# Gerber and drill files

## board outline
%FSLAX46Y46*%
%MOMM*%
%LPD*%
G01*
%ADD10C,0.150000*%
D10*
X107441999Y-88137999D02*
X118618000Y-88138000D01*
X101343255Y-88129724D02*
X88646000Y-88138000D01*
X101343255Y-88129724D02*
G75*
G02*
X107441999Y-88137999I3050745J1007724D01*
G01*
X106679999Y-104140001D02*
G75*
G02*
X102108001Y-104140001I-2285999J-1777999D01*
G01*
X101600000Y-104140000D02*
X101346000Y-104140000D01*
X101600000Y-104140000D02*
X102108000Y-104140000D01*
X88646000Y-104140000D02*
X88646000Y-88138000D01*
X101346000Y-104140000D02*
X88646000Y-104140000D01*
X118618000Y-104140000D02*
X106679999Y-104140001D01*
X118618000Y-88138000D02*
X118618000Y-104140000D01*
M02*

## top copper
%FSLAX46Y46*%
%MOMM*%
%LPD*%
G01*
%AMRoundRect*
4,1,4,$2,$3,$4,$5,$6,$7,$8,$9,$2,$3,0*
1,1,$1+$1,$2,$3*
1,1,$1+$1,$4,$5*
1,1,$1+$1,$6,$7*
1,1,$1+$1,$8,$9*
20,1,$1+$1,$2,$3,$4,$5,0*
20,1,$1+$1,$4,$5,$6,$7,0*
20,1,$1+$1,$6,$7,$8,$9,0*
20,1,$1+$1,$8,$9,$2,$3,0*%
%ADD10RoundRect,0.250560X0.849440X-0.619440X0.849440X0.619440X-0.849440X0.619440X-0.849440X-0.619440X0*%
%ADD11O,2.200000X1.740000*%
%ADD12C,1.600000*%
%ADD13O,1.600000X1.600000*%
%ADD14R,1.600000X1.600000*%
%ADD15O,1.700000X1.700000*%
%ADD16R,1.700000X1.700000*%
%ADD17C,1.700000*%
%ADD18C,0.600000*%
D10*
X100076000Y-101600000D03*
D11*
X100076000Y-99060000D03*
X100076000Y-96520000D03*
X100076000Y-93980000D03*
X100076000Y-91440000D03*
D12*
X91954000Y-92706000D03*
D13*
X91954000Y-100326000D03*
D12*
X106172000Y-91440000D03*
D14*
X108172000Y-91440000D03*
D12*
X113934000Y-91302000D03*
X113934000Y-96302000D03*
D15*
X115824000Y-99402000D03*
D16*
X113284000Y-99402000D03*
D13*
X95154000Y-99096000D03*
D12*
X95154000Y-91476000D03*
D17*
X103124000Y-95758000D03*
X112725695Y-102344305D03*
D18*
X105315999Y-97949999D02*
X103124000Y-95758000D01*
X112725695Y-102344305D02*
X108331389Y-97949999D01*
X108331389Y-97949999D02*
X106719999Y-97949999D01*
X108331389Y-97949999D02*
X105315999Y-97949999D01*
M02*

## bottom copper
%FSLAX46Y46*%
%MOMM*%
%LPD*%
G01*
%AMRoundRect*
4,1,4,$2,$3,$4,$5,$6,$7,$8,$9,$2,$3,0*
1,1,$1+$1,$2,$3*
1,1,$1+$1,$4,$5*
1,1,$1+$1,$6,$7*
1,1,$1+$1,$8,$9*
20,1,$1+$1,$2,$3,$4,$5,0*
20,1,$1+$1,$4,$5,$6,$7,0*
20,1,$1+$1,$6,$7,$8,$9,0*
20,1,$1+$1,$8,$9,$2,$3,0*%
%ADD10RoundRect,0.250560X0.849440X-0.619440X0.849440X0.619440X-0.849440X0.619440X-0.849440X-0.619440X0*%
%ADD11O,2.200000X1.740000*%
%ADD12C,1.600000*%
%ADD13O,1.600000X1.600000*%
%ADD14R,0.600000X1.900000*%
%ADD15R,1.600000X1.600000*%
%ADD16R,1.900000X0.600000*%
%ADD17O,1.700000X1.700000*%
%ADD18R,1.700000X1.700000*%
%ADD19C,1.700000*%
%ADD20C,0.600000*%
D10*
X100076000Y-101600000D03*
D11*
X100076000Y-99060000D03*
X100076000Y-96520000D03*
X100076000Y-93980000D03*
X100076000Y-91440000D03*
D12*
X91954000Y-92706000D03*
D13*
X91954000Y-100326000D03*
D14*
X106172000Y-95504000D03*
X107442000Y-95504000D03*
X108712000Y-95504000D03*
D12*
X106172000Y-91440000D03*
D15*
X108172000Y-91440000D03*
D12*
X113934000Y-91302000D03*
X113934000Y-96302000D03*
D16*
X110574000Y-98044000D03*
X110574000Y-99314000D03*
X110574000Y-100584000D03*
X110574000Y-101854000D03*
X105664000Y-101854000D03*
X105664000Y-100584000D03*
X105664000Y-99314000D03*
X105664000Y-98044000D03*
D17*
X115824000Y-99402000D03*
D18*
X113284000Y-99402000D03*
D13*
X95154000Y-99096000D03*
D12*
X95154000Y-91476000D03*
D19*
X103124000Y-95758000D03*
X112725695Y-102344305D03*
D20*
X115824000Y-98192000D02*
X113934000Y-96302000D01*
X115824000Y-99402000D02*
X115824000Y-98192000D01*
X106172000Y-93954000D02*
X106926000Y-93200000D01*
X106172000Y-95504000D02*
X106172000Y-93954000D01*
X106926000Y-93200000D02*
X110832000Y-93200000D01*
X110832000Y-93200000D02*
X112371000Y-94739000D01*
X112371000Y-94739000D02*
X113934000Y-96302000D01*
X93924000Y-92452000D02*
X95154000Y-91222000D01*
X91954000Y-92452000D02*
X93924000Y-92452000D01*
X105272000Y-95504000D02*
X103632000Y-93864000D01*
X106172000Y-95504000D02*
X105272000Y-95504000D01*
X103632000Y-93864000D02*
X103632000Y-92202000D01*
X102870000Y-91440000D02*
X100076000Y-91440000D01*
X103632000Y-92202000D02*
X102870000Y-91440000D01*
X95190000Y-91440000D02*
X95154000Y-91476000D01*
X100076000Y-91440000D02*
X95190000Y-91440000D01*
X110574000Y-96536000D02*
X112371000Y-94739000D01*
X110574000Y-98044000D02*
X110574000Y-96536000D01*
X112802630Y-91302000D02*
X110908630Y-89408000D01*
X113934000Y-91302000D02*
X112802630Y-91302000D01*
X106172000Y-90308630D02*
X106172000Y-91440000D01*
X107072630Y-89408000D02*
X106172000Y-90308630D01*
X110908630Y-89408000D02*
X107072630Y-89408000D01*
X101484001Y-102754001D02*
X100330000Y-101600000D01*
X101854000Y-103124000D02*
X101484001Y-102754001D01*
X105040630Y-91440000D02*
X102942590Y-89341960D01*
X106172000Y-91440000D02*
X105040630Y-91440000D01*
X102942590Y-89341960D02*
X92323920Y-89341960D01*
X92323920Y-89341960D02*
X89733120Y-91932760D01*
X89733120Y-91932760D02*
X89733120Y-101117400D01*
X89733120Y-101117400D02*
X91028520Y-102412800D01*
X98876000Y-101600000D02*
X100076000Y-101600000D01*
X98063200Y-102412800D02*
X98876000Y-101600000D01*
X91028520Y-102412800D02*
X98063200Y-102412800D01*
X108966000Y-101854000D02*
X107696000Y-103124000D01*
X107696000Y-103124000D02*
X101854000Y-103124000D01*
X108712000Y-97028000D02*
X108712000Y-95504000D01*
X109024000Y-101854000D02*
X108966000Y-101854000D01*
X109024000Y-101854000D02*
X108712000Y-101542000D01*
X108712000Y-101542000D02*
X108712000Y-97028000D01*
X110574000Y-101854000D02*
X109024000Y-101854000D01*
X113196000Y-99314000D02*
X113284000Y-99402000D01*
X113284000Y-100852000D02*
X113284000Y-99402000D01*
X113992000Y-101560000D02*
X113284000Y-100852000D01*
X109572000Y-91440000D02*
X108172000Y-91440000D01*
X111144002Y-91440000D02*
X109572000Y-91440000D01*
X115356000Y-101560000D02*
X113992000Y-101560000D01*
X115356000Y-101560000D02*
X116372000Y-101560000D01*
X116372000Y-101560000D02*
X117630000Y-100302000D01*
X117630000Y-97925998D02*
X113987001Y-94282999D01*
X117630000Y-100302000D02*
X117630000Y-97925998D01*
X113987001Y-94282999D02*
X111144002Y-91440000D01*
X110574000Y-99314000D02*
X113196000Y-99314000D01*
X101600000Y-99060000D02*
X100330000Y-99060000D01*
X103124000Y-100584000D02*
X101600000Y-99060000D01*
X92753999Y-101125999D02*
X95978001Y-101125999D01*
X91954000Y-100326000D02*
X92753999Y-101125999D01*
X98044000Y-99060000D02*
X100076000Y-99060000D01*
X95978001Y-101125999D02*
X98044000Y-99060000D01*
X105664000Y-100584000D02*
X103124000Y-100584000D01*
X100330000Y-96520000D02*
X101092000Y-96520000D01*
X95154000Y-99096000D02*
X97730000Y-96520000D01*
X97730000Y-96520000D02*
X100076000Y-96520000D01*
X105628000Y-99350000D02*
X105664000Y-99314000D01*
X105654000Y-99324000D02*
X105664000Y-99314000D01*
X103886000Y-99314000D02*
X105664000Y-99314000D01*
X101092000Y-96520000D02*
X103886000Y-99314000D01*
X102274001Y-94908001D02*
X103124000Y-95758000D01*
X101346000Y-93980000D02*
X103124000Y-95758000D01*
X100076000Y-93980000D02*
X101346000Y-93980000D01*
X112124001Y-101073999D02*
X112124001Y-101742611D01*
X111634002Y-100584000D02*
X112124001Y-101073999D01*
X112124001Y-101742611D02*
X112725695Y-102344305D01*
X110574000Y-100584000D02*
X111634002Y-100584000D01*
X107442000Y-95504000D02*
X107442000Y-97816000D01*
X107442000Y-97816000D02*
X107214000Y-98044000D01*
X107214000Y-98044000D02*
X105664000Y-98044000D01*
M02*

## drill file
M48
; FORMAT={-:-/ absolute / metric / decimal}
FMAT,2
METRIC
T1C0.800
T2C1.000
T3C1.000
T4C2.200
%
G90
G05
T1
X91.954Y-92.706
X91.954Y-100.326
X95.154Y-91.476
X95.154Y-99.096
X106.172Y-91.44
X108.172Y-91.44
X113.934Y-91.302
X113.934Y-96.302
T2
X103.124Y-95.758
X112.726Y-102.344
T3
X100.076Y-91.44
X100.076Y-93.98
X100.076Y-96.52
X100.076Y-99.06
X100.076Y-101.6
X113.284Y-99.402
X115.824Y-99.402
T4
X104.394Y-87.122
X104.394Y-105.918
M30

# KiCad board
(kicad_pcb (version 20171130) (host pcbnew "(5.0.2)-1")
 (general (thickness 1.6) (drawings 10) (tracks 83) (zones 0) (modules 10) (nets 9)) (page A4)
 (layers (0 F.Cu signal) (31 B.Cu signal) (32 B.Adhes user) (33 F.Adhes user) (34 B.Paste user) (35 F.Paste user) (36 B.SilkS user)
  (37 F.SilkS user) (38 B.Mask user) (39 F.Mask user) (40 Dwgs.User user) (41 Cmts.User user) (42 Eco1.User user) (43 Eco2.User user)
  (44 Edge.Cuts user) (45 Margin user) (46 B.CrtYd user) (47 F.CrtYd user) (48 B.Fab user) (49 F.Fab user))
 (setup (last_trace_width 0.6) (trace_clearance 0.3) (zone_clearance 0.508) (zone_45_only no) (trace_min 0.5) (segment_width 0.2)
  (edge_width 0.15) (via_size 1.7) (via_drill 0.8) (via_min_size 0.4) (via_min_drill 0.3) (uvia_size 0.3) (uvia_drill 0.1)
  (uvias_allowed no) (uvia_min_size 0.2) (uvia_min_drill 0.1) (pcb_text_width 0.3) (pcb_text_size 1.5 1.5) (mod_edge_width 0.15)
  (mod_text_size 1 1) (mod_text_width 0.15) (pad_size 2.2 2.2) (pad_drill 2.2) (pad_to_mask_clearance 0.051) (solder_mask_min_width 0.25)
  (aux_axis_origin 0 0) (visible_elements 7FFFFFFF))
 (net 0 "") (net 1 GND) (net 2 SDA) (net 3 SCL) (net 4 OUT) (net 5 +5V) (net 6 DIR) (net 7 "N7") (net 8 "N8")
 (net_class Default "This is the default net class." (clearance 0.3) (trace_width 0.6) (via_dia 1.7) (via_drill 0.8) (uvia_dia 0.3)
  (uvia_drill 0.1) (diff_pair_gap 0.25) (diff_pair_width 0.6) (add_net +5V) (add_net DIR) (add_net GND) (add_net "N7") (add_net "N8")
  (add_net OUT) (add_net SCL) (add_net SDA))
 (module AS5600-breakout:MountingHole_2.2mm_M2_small (layer F.Cu) (at 104.394 105.918)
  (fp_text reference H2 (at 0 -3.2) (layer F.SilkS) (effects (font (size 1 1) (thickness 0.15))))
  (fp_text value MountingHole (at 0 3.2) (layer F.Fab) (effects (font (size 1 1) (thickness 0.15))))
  (pad 1 np_thru_hole circle (at 0 0) (size 2.2 2.2) (drill 2.2) (layers *.Cu *.Mask)))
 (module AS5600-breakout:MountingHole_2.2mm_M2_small (layer F.Cu) (at 104.394 87.122)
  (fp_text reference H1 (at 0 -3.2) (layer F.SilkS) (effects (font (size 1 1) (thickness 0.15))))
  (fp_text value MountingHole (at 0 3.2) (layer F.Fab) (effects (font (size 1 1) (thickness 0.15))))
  (pad "" np_thru_hole circle (at 0 0) (size 2.2 2.2) (drill 2.2) (layers *.Cu *.Mask)))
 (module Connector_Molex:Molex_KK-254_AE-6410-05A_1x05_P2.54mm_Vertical (layer F.Cu) (at 100.076 101.6 90)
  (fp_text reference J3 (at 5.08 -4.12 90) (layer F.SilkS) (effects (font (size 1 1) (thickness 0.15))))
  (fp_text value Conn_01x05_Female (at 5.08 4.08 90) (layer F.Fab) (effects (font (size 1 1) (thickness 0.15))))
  (pad 1 thru_hole roundrect (at 0 0 90) (size 1.74 2.2) (drill 1) (layers *.Cu *.Mask) (roundrect_rratio 0.144) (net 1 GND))
  (pad 2 thru_hole oval (at 2.54 0 90) (size 1.74 2.2) (drill 1) (layers *.Cu *.Mask) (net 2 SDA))
  (pad 3 thru_hole oval (at 5.08 0 90) (size 1.74 2.2) (drill 1) (layers *.Cu *.Mask) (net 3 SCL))
  (pad 4 thru_hole oval (at 7.62 0 90) (size 1.74 2.2) (drill 1) (layers *.Cu *.Mask) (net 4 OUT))
  (pad 5 thru_hole oval (at 10.16 0 90) (size 1.74 2.2) (drill 1) (layers *.Cu *.Mask) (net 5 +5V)))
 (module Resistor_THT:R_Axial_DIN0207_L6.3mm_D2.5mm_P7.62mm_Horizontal (layer F.Cu) (at 91.954 92.706 270)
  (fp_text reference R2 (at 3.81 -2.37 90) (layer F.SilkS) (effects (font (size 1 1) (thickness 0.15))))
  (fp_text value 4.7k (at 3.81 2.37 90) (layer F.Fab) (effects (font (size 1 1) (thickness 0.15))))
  (pad 1 thru_hole circle (at 0 0 270) (size 1.6 1.6) (drill 0.8) (layers *.Cu *.Mask) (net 5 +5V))
  (pad 2 thru_hole oval (at 7.62 0 270) (size 1.6 1.6) (drill 0.8) (layers *.Cu *.Mask) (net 2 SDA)))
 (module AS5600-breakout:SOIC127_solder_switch (layer B.Cu) (at 106.807 93.049 90)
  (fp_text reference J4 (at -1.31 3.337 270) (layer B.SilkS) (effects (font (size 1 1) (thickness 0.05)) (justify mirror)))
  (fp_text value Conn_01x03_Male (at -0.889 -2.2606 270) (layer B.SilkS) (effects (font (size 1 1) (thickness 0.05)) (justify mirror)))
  (pad 3 smd rect (at -2.455 -0.635 90) (size 1.9 0.6) (layers B.Cu B.Paste B.Mask) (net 5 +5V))
  (pad 2 smd rect (at -2.455 0.635 90) (size 1.9 0.6) (layers B.Cu B.Paste B.Mask) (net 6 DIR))
  (pad 1 smd rect (at -2.455 1.905 90) (size 1.9 0.6) (layers B.Cu B.Paste B.Mask) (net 1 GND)))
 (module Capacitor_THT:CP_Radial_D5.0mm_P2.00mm (layer F.Cu) (at 108.172 91.44 180)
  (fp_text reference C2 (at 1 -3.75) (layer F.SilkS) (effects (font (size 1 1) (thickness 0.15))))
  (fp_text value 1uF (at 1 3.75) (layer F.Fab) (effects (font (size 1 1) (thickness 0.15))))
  (pad 2 thru_hole circle (at 2 0 180) (size 1.6 1.6) (drill 0.8) (layers *.Cu *.Mask) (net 1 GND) (clearance 0.2))
  (pad 1 thru_hole rect (at 0 0 180) (size 1.6 1.6) (drill 0.8) (layers *.Cu *.Mask) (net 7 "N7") (clearance 0.2)))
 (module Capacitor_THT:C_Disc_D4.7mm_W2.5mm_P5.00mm (layer F.Cu) (at 113.934 96.302 90)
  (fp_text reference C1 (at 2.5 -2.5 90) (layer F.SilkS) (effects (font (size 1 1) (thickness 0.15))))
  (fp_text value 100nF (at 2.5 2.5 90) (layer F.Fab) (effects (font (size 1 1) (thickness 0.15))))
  (pad 2 thru_hole circle (at 5 0 90) (size 1.6 1.6) (drill 0.8) (layers *.Cu *.Mask) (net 1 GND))
  (pad 1 thru_hole circle (at 0 0 90) (size 1.6 1.6) (drill 0.8) (layers *.Cu *.Mask) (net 5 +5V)))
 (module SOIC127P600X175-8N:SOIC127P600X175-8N (layer B.Cu) (at 108.119 99.949 180)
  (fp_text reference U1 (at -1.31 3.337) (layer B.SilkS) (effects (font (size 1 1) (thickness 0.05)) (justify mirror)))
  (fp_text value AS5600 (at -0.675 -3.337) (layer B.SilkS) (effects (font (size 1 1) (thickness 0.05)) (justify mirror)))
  (pad 1 smd rect (at -2.455 1.905 180) (size 1.9 0.6) (layers B.Cu B.Paste B.Mask) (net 5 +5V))
  (pad 2 smd rect (at -2.455 0.635 180) (size 1.9 0.6) (layers B.Cu B.Paste B.Mask) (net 7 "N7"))
  (pad 3 smd rect (at -2.455 -0.635 180) (size 1.9 0.6) (layers B.Cu B.Paste B.Mask) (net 4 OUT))
  (pad 4 smd rect (at -2.455 -1.905 180) (size 1.9 0.6) (layers B.Cu B.Paste B.Mask) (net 1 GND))
  (pad 5 smd rect (at 2.455 -1.905 180) (size 1.9 0.6) (layers B.Cu B.Paste B.Mask) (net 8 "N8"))
  (pad 6 smd rect (at 2.455 -0.635 180) (size 1.9 0.6) (layers B.Cu B.Paste B.Mask) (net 2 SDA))
  (pad 7 smd rect (at 2.455 0.635 180) (size 1.9 0.6) (layers B.Cu B.Paste B.Mask) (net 3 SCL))
  (pad 8 smd rect (at 2.455 1.905 180) (size 1.9 0.6) (layers B.Cu B.Paste B.Mask) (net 6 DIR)))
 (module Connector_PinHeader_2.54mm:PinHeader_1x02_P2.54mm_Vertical (layer F.Cu) (at 113.284 99.402 90)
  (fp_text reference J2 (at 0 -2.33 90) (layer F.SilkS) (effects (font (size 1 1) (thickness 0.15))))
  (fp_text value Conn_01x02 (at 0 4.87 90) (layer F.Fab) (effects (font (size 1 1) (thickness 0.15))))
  (pad 2 thru_hole oval (at 0 2.54 90) (size 1.7 1.7) (drill 1) (layers *.Cu *.Mask) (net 5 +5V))
  (pad 1 thru_hole rect (at 0 0 90) (size 1.7 1.7) (drill 1) (layers *.Cu *.Mask) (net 7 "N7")))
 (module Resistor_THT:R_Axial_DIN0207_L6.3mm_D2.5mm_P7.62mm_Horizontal (layer F.Cu) (at 95.154 91.476 270)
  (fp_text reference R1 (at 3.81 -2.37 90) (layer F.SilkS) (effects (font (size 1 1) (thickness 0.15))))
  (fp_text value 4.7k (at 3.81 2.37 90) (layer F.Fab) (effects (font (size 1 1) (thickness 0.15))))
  (pad 2 thru_hole oval (at 7.62 0 270) (size 1.6 1.6) (drill 0.8) (layers *.Cu *.Mask) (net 3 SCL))
  (pad 1 thru_hole circle (at 0 0 270) (size 1.6 1.6) (drill 0.8) (layers *.Cu *.Mask) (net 5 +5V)))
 (gr_line (start 107.441999 88.137999) (end 118.618 88.138) (layer Edge.Cuts) (width 0.15))
 (gr_line (start 101.343255 88.129724) (end 88.646 88.138) (layer Edge.Cuts) (width 0.15))
 (gr_arc (start 104.394 87.122) (end 107.441999 88.137999) (angle -216.714395) (layer Edge.Cuts) (width 0.15))
 (gr_arc (start 104.394 105.918) (end 102.108001 104.140001) (angle -255.7499673) (layer Edge.Cuts) (width 0.15))
 (gr_line (start 101.6 104.14) (end 101.346 104.14) (layer Edge.Cuts) (width 0.15))
 (gr_line (start 101.6 104.14) (end 102.108 104.14) (layer Edge.Cuts) (width 0.15))
 (gr_line (start 88.646 104.14) (end 88.646 88.138) (layer Edge.Cuts) (width 0.15))
 (gr_line (start 101.346 104.14) (end 88.646 104.14) (layer Edge.Cuts) (width 0.15))
 (gr_line (start 118.618 104.14) (end 106.679999 104.140001) (layer Edge.Cuts) (width 0.15))
 (gr_line (start 118.618 88.138) (end 118.618 104.14) (layer Edge.Cuts) (width 0.15))
 (segment (start 115.824 98.192) (end 113.934 96.302) (width 0.6) (layer B.Cu) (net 5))
 (segment (start 115.824 99.402) (end 115.824 98.192) (width 0.6) (layer B.Cu) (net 5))
 (segment (start 106.172 93.954) (end 106.926 93.2) (width 0.6) (layer B.Cu) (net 5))
 (segment (start 106.172 95.504) (end 106.172 93.954) (width 0.6) (layer B.Cu) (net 5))
 (segment (start 106.926 93.2) (end 110.832 93.2) (width 0.6) (layer B.Cu) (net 5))
 (segment (start 110.832 93.2) (end 112.371 94.739) (width 0.6) (layer B.Cu) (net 5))
 (segment (start 112.371 94.739) (end 113.934 96.302) (width 0.6) (layer B.Cu) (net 5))
 (segment (start 93.924 92.452) (end 95.154 91.222) (width 0.6) (layer B.Cu) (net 5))
 (segment (start 91.954 92.452) (end 93.924 92.452) (width 0.6) (layer B.Cu) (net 5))
 (segment (start 105.272 95.504) (end 103.632 93.864) (width 0.6) (layer B.Cu) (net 5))
 (segment (start 106.172 95.504) (end 105.272 95.504) (width 0.6) (layer B.Cu) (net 5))
 (segment (start 103.632 93.864) (end 103.632 92.202) (width 0.6) (layer B.Cu) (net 5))
 (segment (start 102.87 91.44) (end 100.076 91.44) (width 0.6) (layer B.Cu) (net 5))
 (segment (start 103.632 92.202) (end 102.87 91.44) (width 0.6) (layer B.Cu) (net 5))
 (segment (start 95.19 91.44) (end 95.154 91.476) (width 0.6) (layer B.Cu) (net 5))
 (segment (start 100.076 91.44) (end 95.19 91.44) (width 0.6) (layer B.Cu) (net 5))
 (segment (start 110.574 96.536) (end 112.371 94.739) (width 0.6) (layer B.Cu) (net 5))
 (segment (start 110.574 98.044) (end 110.574 96.536) (width 0.6) (layer B.Cu) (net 5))
 (segment (start 112.80263 91.302) (end 110.90863 89.408) (width 0.6) (layer B.Cu) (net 1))
 (segment (start 113.934 91.302) (end 112.80263 91.302) (width 0.6) (layer B.Cu) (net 1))
 (segment (start 106.172 90.30863) (end 106.172 91.44) (width 0.6) (layer B.Cu) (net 1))
 (segment (start 107.07263 89.408) (end 106.172 90.30863) (width 0.6) (layer B.Cu) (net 1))
 (segment (start 110.90863 89.408) (end 107.07263 89.408) (width 0.6) (layer B.Cu) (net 1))
 (segment (start 101.484001 102.754001) (end 100.33 101.6) (width 0.6) (layer B.Cu) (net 1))
 (segment (start 101.854 103.124) (end 101.484001 102.754001) (width 0.6) (layer B.Cu) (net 1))
 (segment (start 105.04063 91.44) (end 102.94259 89.34196) (width 0.6) (layer B.Cu) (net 1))
 (segment (start 106.172 91.44) (end 105.04063 91.44) (width 0.6) (layer B.Cu) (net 1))
 (segment (start 102.94259 89.34196) (end 92.32392 89.34196) (width 0.6) (layer B.Cu) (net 1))
 (segment (start 92.32392 89.34196) (end 89.73312 91.93276) (width 0.6) (layer B.Cu) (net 1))
 (segment (start 89.73312 91.93276) (end 89.73312 101.1174) (width 0.6) (layer B.Cu) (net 1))
 (segment (start 89.73312 101.1174) (end 91.02852 102.4128) (width 0.6) (layer B.Cu) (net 1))
 (segment (start 98.876 101.6) (end 100.076 101.6) (width 0.6) (layer B.Cu) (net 1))
 (segment (start 98.0632 102.4128) (end 98.876 101.6) (width 0.6) (layer B.Cu) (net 1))
 (segment (start 91.02852 102.4128) (end 98.0632 102.4128) (width 0.6) (layer B.Cu) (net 1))
 (segment (start 108.966 101.854) (end 107.696 103.124) (width 0.6) (layer B.Cu) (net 1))
 (segment (start 107.696 103.124) (end 101.854 103.124) (width 0.6) (layer B.Cu) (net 1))
 (segment (start 108.712 97.028) (end 108.712 95.504) (width 0.6) (layer B.Cu) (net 1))
 (segment (start 109.024 101.854) (end 108.966 101.854) (width 0.6) (layer B.Cu) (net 1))
 (segment (start 109.024 101.854) (end 108.712 101.542) (width 0.6) (layer B.Cu) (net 1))
 (segment (start 108.712 101.542) (end 108.712 97.028) (width 0.6) (layer B.Cu) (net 1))
 (segment (start 110.574 101.854) (end 109.024 101.854) (width 0.6) (layer B.Cu) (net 1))
 (segment (start 113.196 99.314) (end 113.284 99.402) (width 0.6) (layer B.Cu) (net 7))
 (segment (start 113.284 100.852) (end 113.284 99.402) (width 0.6) (layer B.Cu) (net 7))
 (segment (start 113.992 101.56) (end 113.284 100.852) (width 0.6) (layer B.Cu) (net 7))
 (segment (start 109.572 91.44) (end 108.172 91.44) (width 0.6) (layer B.Cu) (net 7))
 (segment (start 111.144002 91.44) (end 109.572 91.44) (width 0.6) (layer B.Cu) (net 7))
 (segment (start 115.356 101.56) (end 113.992 101.56) (width 0.6) (layer B.Cu) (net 7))
 (segment (start 115.356 101.56) (end 116.372 101.56) (width 0.6) (layer B.Cu) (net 7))
 (segment (start 116.372 101.56) (end 117.63 100.302) (width 0.6) (layer B.Cu) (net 7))
 (segment (start 117.63 97.925998) (end 113.987001 94.282999) (width 0.6) (layer B.Cu) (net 7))
 (segment (start 117.63 100.302) (end 117.63 97.925998) (width 0.6) (layer B.Cu) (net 7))
 (segment (start 113.987001 94.282999) (end 111.144002 91.44) (width 0.6) (layer B.Cu) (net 7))
 (segment (start 110.574 99.314) (end 113.196 99.314) (width 0.6) (layer B.Cu) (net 7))
 (segment (start 101.6 99.06) (end 100.33 99.06) (width 0.6) (layer B.Cu) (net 2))
 (segment (start 103.124 100.584) (end 101.6 99.06) (width 0.6) (layer B.Cu) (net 2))
 (segment (start 92.753999 101.125999) (end 95.978001 101.125999) (width 0.6) (layer B.Cu) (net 2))
 (segment (start 91.954 100.326) (end 92.753999 101.125999) (width 0.6) (layer B.Cu) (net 2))
 (segment (start 98.044 99.06) (end 100.076 99.06) (width 0.6) (layer B.Cu) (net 2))
 (segment (start 95.978001 101.125999) (end 98.044 99.06) (width 0.6) (layer B.Cu) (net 2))
 (segment (start 105.664 100.584) (end 103.124 100.584) (width 0.6) (layer B.Cu) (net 2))
 (segment (start 100.33 96.52) (end 101.092 96.52) (width 0.6) (layer B.Cu) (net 3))
 (segment (start 95.154 99.096) (end 97.73 96.52) (width 0.6) (layer B.Cu) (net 3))
 (segment (start 97.73 96.52) (end 100.076 96.52) (width 0.6) (layer B.Cu) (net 3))
 (segment (start 105.628 99.35) (end 105.664 99.314) (width 0.6) (layer B.Cu) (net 3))
 (segment (start 105.654 99.324) (end 105.664 99.314) (width 0.6) (layer B.Cu) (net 3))
 (segment (start 103.886 99.314) (end 105.664 99.314) (width 0.6) (layer B.Cu) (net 3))
 (segment (start 101.092 96.52) (end 103.886 99.314) (width 0.6) (layer B.Cu) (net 3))
 (via (at 103.124 95.758) (size 1.7) (drill 1) (layers F.Cu B.Cu) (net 4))
 (segment (start 102.274001 94.908001) (end 103.124 95.758) (width 0.6) (layer B.Cu) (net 4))
 (segment (start 101.346 93.98) (end 103.124 95.758) (width 0.6) (layer B.Cu) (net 4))
 (segment (start 100.076 93.98) (end 101.346 93.98) (width 0.6) (layer B.Cu) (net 4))
 (segment (start 105.315999 97.949999) (end 103.124 95.758) (width 0.6) (layer F.Cu) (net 4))
 (segment (start 112.124001 101.073999) (end 112.124001 101.742611) (width 0.6) (layer B.Cu) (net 4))
 (segment (start 112.725695 102.344305) (end 108.331389 97.949999) (width 0.6) (layer F.Cu) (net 4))
 (segment (start 111.634002 100.584) (end 112.124001 101.073999) (width 0.6) (layer B.Cu) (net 4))
 (segment (start 112.124001 101.742611) (end 112.725695 102.344305) (width 0.6) (layer B.Cu) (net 4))
 (via (at 112.725695 102.344305) (size 1.7) (drill 1) (layers F.Cu B.Cu) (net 4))
 (segment (start 110.574 100.584) (end 111.634002 100.584) (width 0.6) (layer B.Cu) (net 4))
 (segment (start 107.442 95.504) (end 107.442 97.816) (width 0.6) (layer B.Cu) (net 6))
 (segment (start 107.442 97.816) (end 107.214 98.044) (width 0.6) (layer B.Cu) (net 6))
 (segment (start 107.214 98.044) (end 105.664 98.044) (width 0.6) (layer B.Cu) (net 6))
 (segment (start 108.331389 97.949999) (end 106.719999 97.949999) (width 0.6) (layer F.Cu) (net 4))
 (segment (start 108.331389 97.949999) (end 105.315999 97.949999) (width 0.6) (layer F.Cu) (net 4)))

